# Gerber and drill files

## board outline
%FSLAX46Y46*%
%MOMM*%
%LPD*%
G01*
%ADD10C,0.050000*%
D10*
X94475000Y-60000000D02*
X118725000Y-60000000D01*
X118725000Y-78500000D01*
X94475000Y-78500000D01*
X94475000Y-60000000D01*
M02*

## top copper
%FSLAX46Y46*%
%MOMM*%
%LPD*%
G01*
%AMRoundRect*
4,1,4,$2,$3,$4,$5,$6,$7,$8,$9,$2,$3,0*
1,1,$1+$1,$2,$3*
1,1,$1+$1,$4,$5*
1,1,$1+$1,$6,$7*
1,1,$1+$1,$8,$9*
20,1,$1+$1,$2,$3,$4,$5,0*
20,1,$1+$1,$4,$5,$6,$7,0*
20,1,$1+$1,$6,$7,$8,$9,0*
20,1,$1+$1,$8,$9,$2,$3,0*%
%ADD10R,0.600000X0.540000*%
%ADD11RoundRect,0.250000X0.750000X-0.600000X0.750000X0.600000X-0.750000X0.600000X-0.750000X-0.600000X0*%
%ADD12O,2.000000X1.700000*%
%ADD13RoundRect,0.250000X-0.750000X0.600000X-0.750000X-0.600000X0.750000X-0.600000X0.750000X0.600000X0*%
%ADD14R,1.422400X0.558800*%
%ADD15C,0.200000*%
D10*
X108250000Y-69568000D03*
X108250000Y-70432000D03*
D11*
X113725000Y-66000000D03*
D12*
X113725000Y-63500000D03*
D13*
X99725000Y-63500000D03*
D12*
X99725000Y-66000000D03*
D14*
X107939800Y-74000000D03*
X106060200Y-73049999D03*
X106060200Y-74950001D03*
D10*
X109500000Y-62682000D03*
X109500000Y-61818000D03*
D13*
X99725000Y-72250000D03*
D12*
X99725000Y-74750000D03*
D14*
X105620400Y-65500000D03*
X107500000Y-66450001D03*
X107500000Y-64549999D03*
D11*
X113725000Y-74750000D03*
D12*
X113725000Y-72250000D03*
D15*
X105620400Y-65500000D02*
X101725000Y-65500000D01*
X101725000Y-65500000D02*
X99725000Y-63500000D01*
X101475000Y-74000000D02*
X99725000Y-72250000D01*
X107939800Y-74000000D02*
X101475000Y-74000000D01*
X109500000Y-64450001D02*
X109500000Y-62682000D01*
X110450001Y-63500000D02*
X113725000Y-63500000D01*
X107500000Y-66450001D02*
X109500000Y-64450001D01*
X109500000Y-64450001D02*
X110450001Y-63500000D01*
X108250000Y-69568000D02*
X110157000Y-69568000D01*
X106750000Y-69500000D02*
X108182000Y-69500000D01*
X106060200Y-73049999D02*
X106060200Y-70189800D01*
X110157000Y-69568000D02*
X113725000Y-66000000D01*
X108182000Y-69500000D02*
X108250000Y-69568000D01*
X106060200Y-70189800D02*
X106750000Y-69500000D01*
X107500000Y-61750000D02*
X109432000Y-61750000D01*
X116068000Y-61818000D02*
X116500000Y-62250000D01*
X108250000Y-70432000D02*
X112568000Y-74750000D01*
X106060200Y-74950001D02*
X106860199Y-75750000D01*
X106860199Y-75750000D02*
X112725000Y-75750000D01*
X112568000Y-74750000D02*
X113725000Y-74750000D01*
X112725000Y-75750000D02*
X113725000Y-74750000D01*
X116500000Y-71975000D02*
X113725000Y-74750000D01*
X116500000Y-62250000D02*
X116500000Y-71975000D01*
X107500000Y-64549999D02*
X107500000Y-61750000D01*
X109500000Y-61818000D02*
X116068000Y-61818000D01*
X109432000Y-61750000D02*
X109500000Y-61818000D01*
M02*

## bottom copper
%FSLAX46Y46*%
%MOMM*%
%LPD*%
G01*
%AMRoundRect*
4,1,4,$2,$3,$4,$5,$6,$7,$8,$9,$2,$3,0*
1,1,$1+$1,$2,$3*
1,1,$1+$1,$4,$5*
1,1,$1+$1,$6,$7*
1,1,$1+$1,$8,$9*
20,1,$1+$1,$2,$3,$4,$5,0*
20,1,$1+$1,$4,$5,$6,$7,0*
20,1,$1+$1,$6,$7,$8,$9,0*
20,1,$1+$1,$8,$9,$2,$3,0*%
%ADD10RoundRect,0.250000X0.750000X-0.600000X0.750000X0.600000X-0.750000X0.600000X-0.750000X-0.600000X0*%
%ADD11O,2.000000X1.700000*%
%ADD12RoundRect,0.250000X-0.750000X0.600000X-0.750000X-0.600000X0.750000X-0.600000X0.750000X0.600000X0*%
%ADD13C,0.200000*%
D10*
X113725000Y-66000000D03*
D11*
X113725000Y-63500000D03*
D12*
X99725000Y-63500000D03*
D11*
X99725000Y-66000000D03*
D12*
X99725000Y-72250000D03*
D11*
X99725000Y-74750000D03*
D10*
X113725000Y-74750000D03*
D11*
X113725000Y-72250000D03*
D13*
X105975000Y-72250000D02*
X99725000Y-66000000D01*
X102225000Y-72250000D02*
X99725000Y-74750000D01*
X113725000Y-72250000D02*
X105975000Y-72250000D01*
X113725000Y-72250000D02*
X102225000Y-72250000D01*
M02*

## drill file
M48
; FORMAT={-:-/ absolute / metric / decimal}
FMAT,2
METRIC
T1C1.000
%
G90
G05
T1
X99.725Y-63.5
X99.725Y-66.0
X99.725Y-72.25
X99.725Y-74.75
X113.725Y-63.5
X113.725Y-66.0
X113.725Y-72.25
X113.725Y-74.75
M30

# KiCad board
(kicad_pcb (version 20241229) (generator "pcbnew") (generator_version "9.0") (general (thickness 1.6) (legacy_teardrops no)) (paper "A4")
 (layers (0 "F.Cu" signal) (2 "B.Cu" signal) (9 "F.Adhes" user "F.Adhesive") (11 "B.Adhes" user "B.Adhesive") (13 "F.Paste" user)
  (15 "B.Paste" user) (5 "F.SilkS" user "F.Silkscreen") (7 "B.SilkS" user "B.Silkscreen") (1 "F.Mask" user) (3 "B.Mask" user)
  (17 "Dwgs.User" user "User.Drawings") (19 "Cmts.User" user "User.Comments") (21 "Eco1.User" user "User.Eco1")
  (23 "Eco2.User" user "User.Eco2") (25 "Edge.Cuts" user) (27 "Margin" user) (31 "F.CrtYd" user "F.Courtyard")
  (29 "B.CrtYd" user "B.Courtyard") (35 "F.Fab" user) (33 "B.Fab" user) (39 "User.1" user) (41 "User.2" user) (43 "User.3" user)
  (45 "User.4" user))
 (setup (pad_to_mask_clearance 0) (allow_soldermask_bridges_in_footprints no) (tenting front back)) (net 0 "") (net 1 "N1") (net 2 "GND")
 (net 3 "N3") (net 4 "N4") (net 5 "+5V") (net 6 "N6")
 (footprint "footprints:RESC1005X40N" (layer "F.Cu") (at 108.25 70 -90)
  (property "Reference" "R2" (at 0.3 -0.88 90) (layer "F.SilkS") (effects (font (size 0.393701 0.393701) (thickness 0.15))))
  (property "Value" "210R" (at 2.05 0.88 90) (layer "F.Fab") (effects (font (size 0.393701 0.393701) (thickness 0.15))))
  (pad "1" smd rect (at -0.432 0 270) (size 0.54 0.6) (layers "F.Cu" "F.Mask" "F.Paste") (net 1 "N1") (solder_mask_margin 0.102))
  (pad "2" smd rect (at 0.432 0 270) (size 0.54 0.6) (layers "F.Cu" "F.Mask" "F.Paste") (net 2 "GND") (solder_mask_margin 0.102)))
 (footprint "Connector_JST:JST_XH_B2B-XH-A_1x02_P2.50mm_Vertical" (layer "F.Cu") (at 113.725 66 90)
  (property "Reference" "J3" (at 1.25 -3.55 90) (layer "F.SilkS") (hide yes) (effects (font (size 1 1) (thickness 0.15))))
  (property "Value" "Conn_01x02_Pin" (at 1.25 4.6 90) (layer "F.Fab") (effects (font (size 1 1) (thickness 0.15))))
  (pad "1" thru_hole roundrect (at 0 0 90) (size 1.7 2) (drill 1) (layers "*.Cu" "*.Mask") (remove_unused_layers no)
   (roundrect_rratio 0.147059) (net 1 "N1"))
  (pad "2" thru_hole oval (at 2.5 0 90) (size 1.7 2) (drill 1) (layers "*.Cu" "*.Mask") (remove_unused_layers no) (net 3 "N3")))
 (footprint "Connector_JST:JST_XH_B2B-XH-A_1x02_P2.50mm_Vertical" (layer "F.Cu") (at 99.725 63.5 -90)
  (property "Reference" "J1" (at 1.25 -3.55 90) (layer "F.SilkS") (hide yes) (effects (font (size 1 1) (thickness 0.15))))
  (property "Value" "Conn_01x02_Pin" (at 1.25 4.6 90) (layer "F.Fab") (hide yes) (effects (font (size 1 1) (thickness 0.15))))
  (pad "1" thru_hole roundrect (at 0 0 270) (size 1.7 2) (drill 1) (layers "*.Cu" "*.Mask") (remove_unused_layers no)
   (roundrect_rratio 0.147059) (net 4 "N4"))
  (pad "2" thru_hole oval (at 2.5 0 270) (size 1.7 2) (drill 1) (layers "*.Cu" "*.Mask") (remove_unused_layers no) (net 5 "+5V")))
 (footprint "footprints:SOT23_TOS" (layer "F.Cu") (at 107 74 -90)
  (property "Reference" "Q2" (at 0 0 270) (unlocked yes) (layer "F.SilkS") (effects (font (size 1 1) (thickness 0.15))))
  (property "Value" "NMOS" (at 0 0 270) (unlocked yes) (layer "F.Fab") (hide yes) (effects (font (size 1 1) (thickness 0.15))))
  (pad "1" smd rect (at 0 -0.9398 270) (size 0.5588 1.4224) (layers "F.Cu" "F.Mask" "F.Paste") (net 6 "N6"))
  (pad "2" smd rect (at -0.950001 0.9398 270) (size 0.5588 1.4224) (layers "F.Cu" "F.Mask" "F.Paste") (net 1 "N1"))
  (pad "3" smd rect (at 0.950001 0.9398 270) (size 0.5588 1.4224) (layers "F.Cu" "F.Mask" "F.Paste") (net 2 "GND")))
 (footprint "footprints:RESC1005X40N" (layer "F.Cu") (at 109.5 62.25 90)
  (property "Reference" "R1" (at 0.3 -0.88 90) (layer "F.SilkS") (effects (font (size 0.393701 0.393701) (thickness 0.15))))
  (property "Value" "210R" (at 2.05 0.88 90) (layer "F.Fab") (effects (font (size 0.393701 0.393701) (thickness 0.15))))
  (pad "1" smd rect (at -0.432 0 90) (size 0.54 0.6) (layers "F.Cu" "F.Mask" "F.Paste") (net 3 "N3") (solder_mask_margin 0.102))
  (pad "2" smd rect (at 0.432 0 90) (size 0.54 0.6) (layers "F.Cu" "F.Mask" "F.Paste") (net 2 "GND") (solder_mask_margin 0.102)))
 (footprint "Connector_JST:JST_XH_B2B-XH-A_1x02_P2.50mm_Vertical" (layer "F.Cu") (at 99.725 72.25 -90)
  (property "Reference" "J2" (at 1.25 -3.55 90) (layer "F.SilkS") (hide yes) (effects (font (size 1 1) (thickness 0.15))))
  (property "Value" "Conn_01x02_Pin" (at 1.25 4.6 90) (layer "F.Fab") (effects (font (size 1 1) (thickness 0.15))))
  (pad "1" thru_hole roundrect (at 0 0 270) (size 1.7 2) (drill 1) (layers "*.Cu" "*.Mask") (remove_unused_layers no)
   (roundrect_rratio 0.147059) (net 6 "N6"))
  (pad "2" thru_hole oval (at 2.5 0 270) (size 1.7 2) (drill 1) (layers "*.Cu" "*.Mask") (remove_unused_layers no) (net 5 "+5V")))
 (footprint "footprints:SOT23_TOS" (layer "F.Cu") (at 106.5602 65.5 90)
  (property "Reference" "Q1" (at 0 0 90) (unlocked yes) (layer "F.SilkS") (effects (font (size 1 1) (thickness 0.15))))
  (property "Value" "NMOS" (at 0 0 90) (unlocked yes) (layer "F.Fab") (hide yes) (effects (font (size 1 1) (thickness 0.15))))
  (pad "1" smd rect (at 0 -0.9398 90) (size 0.5588 1.4224) (layers "F.Cu" "F.Mask" "F.Paste") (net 4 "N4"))
  (pad "2" smd rect (at -0.950001 0.9398 90) (size 0.5588 1.4224) (layers "F.Cu" "F.Mask" "F.Paste") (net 3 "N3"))
  (pad "3" smd rect (at 0.950001 0.9398 90) (size 0.5588 1.4224) (layers "F.Cu" "F.Mask" "F.Paste") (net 2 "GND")))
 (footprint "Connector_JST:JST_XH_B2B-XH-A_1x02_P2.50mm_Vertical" (layer "F.Cu") (at 113.725 74.75 90)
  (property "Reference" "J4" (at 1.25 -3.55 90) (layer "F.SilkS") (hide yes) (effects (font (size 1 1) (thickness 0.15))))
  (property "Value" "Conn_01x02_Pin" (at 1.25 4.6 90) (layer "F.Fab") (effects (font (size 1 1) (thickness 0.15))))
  (pad "1" thru_hole roundrect (at 0 0 90) (size 1.7 2) (drill 1) (layers "*.Cu" "*.Mask") (remove_unused_layers no)
   (roundrect_rratio 0.147059) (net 2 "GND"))
  (pad "2" thru_hole oval (at 2.5 0 90) (size 1.7 2) (drill 1) (layers "*.Cu" "*.Mask") (remove_unused_layers no) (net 5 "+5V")))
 (gr_rect (start 94.475 60) (end 118.725 78.5) (stroke (width 0.05) (type default)) (fill no) (layer "Edge.Cuts"))
 (segment (start 105.6204 65.5) (end 101.725 65.5) (width 0.2) (layer "F.Cu") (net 4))
 (segment (start 101.725 65.5) (end 99.725 63.5) (width 0.2) (layer "F.Cu") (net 4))
 (segment (start 105.975 72.25) (end 99.725 66) (width 0.2) (layer "B.Cu") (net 5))
 (segment (start 102.225 72.25) (end 99.725 74.75) (width 0.2) (layer "B.Cu") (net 5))
 (segment (start 113.725 72.25) (end 105.975 72.25) (width 0.2) (layer "B.Cu") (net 5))
 (segment (start 113.725 72.25) (end 102.225 72.25) (width 0.2) (layer "B.Cu") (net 5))
 (segment (start 101.475 74) (end 99.725 72.25) (width 0.2) (layer "F.Cu") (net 6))
 (segment (start 107.9398 74) (end 101.475 74) (width 0.2) (layer "F.Cu") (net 6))
 (segment (start 109.5 64.450001) (end 109.5 62.682) (width 0.2) (layer "F.Cu") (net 3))
 (segment (start 110.450001 63.5) (end 113.725 63.5) (width 0.2) (layer "F.Cu") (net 3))
 (segment (start 107.5 66.450001) (end 109.5 64.450001) (width 0.2) (layer "F.Cu") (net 3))
 (segment (start 109.5 64.450001) (end 110.450001 63.5) (width 0.2) (layer "F.Cu") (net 3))
 (segment (start 108.25 69.568) (end 110.157 69.568) (width 0.2) (layer "F.Cu") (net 1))
 (segment (start 106.75 69.5) (end 108.182 69.5) (width 0.2) (layer "F.Cu") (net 1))
 (segment (start 106.0602 73.049999) (end 106.0602 70.1898) (width 0.2) (layer "F.Cu") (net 1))
 (segment (start 110.157 69.568) (end 113.725 66) (width 0.2) (layer "F.Cu") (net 1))
 (segment (start 108.182 69.5) (end 108.25 69.568) (width 0.2) (layer "F.Cu") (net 1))
 (segment (start 106.0602 70.1898) (end 106.75 69.5) (width 0.2) (layer "F.Cu") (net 1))
 (segment (start 107.5 61.75) (end 109.432 61.75) (width 0.2) (layer "F.Cu") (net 2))
 (segment (start 116.068 61.818) (end 116.5 62.25) (width 0.2) (layer "F.Cu") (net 2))
 (segment (start 108.25 70.432) (end 112.568 74.75) (width 0.2) (layer "F.Cu") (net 2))
 (segment (start 106.0602 74.950001) (end 106.860199 75.75) (width 0.2) (layer "F.Cu") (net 2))
 (segment (start 106.860199 75.75) (end 112.725 75.75) (width 0.2) (layer "F.Cu") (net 2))
 (segment (start 112.568 74.75) (end 113.725 74.75) (width 0.2) (layer "F.Cu") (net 2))
 (segment (start 112.725 75.75) (end 113.725 74.75) (width 0.2) (layer "F.Cu") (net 2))
 (segment (start 116.5 71.975) (end 113.725 74.75) (width 0.2) (layer "F.Cu") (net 2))
 (segment (start 116.5 62.25) (end 116.5 71.975) (width 0.2) (layer "F.Cu") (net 2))
 (segment (start 107.5 64.549999) (end 107.5 61.75) (width 0.2) (layer "F.Cu") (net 2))
 (segment (start 109.5 61.818) (end 116.068 61.818) (width 0.2) (layer "F.Cu") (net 2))
 (segment (start 109.432 61.75) (end 109.5 61.818) (width 0.2) (layer "F.Cu") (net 2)))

